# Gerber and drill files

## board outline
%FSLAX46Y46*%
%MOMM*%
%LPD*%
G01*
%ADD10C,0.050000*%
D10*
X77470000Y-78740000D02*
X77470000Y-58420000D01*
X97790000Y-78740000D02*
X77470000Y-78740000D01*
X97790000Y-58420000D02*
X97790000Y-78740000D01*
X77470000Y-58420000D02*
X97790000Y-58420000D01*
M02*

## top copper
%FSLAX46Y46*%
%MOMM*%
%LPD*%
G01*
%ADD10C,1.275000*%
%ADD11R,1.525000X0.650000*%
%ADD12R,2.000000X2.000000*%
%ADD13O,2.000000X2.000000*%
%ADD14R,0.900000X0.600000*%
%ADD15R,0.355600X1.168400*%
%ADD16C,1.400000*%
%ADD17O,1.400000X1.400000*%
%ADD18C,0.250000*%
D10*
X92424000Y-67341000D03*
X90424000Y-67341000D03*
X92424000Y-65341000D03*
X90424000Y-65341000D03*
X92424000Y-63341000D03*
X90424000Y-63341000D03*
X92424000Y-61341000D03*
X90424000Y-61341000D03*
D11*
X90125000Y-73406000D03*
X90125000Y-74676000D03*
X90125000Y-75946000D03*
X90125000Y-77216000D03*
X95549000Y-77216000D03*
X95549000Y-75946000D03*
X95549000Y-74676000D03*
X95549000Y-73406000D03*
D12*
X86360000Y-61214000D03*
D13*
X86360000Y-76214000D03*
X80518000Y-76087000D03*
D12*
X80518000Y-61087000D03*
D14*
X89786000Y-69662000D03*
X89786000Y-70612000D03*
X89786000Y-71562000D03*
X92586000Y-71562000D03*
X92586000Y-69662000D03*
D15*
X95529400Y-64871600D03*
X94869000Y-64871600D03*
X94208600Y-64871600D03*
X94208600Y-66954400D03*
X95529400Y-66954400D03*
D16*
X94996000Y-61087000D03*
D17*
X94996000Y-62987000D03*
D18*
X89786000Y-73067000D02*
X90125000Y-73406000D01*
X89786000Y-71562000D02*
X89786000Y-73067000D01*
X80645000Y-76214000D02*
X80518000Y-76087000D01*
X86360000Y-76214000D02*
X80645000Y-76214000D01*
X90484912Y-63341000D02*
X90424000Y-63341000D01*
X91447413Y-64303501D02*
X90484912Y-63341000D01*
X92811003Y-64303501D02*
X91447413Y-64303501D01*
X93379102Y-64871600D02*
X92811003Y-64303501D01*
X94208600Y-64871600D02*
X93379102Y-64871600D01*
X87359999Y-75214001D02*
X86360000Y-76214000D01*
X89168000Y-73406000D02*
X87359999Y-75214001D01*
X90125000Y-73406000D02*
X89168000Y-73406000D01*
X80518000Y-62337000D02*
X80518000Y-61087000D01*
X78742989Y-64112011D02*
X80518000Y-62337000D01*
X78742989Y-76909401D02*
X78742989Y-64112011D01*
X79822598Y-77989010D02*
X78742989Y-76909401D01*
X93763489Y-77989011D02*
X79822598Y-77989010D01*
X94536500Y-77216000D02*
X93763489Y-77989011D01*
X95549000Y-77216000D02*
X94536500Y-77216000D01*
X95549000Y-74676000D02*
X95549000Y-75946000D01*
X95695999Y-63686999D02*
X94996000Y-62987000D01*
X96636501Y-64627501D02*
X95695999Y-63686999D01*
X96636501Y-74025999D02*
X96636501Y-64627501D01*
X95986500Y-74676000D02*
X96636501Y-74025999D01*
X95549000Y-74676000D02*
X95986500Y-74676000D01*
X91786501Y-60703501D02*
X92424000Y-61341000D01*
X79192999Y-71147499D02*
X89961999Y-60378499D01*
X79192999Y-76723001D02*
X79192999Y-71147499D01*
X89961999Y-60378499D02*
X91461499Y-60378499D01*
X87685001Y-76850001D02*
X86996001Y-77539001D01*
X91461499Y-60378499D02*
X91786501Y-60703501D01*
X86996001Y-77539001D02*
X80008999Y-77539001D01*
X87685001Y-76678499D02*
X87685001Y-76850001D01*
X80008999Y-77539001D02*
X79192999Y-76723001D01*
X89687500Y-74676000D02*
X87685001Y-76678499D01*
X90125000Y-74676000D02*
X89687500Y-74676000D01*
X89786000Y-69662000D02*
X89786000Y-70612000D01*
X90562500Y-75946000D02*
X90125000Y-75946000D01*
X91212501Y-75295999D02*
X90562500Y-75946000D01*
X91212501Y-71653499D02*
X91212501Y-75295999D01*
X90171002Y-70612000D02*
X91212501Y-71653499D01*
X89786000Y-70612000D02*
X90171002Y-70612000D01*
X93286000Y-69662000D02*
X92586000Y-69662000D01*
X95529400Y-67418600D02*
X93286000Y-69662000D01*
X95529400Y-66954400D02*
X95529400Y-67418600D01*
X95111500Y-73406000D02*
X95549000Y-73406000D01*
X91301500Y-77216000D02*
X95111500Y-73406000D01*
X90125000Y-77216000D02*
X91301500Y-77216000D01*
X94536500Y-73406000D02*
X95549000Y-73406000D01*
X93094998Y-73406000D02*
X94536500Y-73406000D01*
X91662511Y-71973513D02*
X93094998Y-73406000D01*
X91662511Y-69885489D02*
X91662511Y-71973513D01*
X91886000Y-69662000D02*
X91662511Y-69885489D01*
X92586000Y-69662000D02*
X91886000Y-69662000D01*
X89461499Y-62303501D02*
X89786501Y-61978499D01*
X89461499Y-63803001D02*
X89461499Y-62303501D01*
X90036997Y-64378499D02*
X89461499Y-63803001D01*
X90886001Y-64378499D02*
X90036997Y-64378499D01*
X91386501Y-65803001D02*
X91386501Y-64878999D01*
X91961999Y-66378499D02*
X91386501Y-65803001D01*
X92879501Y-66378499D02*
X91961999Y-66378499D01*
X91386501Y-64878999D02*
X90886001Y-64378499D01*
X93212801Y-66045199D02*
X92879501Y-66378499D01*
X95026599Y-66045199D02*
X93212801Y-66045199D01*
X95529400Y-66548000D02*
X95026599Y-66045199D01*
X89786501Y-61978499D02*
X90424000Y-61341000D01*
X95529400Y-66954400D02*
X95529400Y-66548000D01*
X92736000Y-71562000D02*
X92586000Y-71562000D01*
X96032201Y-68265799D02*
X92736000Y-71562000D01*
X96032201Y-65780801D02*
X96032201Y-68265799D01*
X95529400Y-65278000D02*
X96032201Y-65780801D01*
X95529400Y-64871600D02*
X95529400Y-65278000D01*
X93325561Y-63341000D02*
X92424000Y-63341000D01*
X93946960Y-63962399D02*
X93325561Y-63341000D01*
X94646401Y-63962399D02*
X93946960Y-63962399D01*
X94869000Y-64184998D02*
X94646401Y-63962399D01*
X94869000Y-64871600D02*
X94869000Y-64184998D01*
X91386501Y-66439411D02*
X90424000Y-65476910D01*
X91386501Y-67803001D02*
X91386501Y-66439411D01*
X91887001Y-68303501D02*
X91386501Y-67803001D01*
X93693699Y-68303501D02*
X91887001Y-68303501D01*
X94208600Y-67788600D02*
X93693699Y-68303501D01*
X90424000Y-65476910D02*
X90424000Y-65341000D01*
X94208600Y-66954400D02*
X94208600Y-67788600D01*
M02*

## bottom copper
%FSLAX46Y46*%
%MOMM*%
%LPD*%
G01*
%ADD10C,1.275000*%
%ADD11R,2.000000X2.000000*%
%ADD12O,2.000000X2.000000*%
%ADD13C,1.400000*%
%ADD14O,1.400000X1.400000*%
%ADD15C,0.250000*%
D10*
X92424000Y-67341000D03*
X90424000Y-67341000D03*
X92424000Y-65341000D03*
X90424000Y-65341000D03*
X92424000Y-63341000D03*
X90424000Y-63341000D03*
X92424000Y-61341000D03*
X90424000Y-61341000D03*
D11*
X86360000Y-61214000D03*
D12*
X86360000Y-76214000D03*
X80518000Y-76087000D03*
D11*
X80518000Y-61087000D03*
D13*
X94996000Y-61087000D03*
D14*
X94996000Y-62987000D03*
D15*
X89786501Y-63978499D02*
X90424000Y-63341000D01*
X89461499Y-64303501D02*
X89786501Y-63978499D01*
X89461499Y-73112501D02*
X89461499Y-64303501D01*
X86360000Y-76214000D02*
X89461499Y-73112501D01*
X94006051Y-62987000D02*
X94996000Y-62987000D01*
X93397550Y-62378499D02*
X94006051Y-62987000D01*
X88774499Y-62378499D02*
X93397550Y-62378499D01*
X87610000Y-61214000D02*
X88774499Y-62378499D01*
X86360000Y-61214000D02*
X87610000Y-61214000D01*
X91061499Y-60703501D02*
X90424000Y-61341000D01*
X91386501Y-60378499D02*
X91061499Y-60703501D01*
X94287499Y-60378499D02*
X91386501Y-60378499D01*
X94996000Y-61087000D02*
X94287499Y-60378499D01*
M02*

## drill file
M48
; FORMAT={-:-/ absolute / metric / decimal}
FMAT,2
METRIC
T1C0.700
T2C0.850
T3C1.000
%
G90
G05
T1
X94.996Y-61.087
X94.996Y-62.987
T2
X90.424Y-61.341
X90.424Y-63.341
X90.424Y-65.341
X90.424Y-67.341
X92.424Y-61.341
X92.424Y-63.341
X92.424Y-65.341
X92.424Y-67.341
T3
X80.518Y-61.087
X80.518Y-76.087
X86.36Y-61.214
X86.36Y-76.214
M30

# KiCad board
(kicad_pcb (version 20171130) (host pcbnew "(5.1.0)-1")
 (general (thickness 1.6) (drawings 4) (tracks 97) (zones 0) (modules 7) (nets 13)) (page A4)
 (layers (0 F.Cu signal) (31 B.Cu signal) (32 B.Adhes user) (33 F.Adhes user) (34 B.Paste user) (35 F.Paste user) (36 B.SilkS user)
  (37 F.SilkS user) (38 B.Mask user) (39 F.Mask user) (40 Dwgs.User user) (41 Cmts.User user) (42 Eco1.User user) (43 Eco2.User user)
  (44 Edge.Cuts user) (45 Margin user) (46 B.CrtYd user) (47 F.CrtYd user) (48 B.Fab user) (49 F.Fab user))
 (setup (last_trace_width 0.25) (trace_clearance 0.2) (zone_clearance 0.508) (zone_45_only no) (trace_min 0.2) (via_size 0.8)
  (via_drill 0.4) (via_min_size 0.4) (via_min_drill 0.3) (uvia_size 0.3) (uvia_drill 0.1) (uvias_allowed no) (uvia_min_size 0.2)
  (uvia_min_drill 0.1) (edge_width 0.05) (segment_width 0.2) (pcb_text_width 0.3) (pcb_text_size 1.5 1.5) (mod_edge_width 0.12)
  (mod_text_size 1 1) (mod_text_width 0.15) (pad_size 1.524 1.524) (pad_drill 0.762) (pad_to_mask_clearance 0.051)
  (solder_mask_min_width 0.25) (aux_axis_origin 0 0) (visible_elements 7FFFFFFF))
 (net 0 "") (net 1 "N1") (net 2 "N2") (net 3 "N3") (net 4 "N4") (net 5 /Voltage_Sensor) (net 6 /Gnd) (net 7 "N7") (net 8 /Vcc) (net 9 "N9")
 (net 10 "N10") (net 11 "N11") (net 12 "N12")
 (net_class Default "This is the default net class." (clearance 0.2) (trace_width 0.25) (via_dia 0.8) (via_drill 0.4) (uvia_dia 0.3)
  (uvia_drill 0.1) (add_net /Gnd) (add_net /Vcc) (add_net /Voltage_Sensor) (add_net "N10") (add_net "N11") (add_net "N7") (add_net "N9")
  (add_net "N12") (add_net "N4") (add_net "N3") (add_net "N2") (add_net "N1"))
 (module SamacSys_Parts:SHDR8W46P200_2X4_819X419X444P (layer F.Cu) (at 90.424 61.341 270)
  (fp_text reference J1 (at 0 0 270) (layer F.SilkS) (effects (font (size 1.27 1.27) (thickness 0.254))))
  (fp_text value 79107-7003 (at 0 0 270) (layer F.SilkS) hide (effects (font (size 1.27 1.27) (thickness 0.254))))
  (pad 8 thru_hole circle (at 6 -2 270) (size 1.275 1.275) (drill 0.85) (layers *.Cu *.Mask) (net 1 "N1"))
  (pad 7 thru_hole circle (at 6 0 270) (size 1.275 1.275) (drill 0.85) (layers *.Cu *.Mask) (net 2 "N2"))
  (pad 6 thru_hole circle (at 4 -2 270) (size 1.275 1.275) (drill 0.85) (layers *.Cu *.Mask) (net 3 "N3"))
  (pad 5 thru_hole circle (at 4 0 270) (size 1.275 1.275) (drill 0.85) (layers *.Cu *.Mask) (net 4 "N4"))
  (pad 4 thru_hole circle (at 2 -2 270) (size 1.275 1.275) (drill 0.85) (layers *.Cu *.Mask) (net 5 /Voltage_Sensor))
  (pad 3 thru_hole circle (at 2 0 270) (size 1.275 1.275) (drill 0.85) (layers *.Cu *.Mask) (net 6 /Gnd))
  (pad 2 thru_hole circle (at 0 -2 270) (size 1.275 1.275) (drill 0.85) (layers *.Cu *.Mask) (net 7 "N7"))
  (pad 1 thru_hole circle (at 0 0 270) (size 1.275 1.275) (drill 0.85) (layers *.Cu *.Mask) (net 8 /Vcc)))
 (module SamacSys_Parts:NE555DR (layer F.Cu) (at 92.837 75.311)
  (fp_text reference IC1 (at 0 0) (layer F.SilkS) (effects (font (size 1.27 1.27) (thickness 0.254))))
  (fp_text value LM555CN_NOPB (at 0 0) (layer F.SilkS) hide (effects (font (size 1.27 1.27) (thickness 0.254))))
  (pad 1 smd rect (at -2.712 -1.905 90) (size 0.65 1.525) (layers F.Cu F.Paste) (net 6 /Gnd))
  (pad 2 smd rect (at -2.712 -0.635 90) (size 0.65 1.525) (layers F.Cu F.Paste) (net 7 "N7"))
  (pad 3 smd rect (at -2.712 0.635 90) (size 0.65 1.525) (layers F.Cu F.Paste) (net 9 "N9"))
  (pad 4 smd rect (at -2.712 1.905 90) (size 0.65 1.525) (layers F.Cu F.Paste) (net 8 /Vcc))
  (pad 5 smd rect (at 2.712 1.905 90) (size 0.65 1.525) (layers F.Cu F.Paste) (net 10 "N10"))
  (pad 6 smd rect (at 2.712 0.635 90) (size 0.65 1.525) (layers F.Cu F.Paste) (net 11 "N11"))
  (pad 7 smd rect (at 2.712 -0.635 90) (size 0.65 1.525) (layers F.Cu F.Paste) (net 11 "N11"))
  (pad 8 smd rect (at 2.712 -1.905 90) (size 0.65 1.525) (layers F.Cu F.Paste) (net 8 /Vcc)))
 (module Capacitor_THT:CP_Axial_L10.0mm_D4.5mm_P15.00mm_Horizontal (layer F.Cu) (at 86.36 61.214 270)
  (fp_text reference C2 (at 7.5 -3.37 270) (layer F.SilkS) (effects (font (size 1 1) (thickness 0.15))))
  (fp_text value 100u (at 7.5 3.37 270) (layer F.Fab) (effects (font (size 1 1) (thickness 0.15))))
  (pad 1 thru_hole rect (at 0 0 270) (size 2 2) (drill 1) (layers *.Cu *.Mask) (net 11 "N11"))
  (pad 2 thru_hole oval (at 15 0 270) (size 2 2) (drill 1) (layers *.Cu *.Mask) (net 6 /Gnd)))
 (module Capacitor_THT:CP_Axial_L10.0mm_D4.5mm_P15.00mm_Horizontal (layer F.Cu) (at 80.518 61.087 270)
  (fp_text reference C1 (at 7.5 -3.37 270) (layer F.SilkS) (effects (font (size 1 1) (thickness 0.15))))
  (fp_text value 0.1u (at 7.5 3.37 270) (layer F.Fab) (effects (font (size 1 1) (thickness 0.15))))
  (pad 2 thru_hole oval (at 15 0 270) (size 2 2) (drill 1) (layers *.Cu *.Mask) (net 6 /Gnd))
  (pad 1 thru_hole rect (at 0 0 270) (size 2 2) (drill 1) (layers *.Cu *.Mask) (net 10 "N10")))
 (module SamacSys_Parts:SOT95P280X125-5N (layer F.Cu) (at 91.186 70.612)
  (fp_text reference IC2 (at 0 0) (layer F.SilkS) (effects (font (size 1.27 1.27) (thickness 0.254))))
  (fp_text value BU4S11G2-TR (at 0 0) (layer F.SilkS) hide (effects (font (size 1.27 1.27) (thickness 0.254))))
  (pad 1 smd rect (at -1.4 -0.95 90) (size 0.6 0.9) (layers F.Cu F.Paste F.Mask) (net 9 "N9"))
  (pad 2 smd rect (at -1.4 0 90) (size 0.6 0.9) (layers F.Cu F.Paste F.Mask) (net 9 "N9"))
  (pad 3 smd rect (at -1.4 0.95 90) (size 0.6 0.9) (layers F.Cu F.Paste F.Mask) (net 6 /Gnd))
  (pad 4 smd rect (at 1.4 0.95 90) (size 0.6 0.9) (layers F.Cu F.Paste F.Mask) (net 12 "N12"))
  (pad 5 smd rect (at 1.4 -0.95 90) (size 0.6 0.9) (layers F.Cu F.Paste F.Mask) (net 8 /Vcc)))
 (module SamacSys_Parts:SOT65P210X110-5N (layer F.Cu) (at 94.869 65.913 270)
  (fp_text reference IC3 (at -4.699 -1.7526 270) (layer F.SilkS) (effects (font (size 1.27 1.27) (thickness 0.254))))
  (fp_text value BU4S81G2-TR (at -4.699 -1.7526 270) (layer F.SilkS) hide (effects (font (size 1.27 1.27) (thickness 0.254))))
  (pad 1 smd rect (at -1.0414 -0.6604) (size 0.3556 1.1684) (layers F.Cu F.Paste F.Mask) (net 12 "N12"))
  (pad 2 smd rect (at -1.0414 0) (size 0.3556 1.1684) (layers F.Cu F.Paste F.Mask) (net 5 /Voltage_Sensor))
  (pad 3 smd rect (at -1.0414 0.6604) (size 0.3556 1.1684) (layers F.Cu F.Paste F.Mask) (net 6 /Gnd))
  (pad 4 smd rect (at 1.0414 0.6604) (size 0.3556 1.1684) (layers F.Cu F.Paste F.Mask) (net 4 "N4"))
  (pad 5 smd rect (at 1.0414 -0.6604) (size 0.3556 1.1684) (layers F.Cu F.Paste F.Mask) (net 8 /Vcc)))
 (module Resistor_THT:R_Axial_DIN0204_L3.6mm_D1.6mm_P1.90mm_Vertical (layer F.Cu) (at 94.996 61.087 270)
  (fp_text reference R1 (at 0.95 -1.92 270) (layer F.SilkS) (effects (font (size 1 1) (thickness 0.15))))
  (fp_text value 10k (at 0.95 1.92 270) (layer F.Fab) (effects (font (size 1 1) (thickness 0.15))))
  (pad 1 thru_hole circle (at 0 0 270) (size 1.4 1.4) (drill 0.7) (layers *.Cu *.Mask) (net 8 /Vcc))
  (pad 2 thru_hole oval (at 1.9 0 270) (size 1.4 1.4) (drill 0.7) (layers *.Cu *.Mask) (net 11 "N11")))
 (gr_line (start 77.47 78.74) (end 77.47 58.42) (layer Edge.Cuts) (width 0.05))
 (gr_line (start 97.79 78.74) (end 77.47 78.74) (layer Edge.Cuts) (width 0.05))
 (gr_line (start 97.79 58.42) (end 97.79 78.74) (layer Edge.Cuts) (width 0.05))
 (gr_line (start 77.47 58.42) (end 97.79 58.42) (layer Edge.Cuts) (width 0.05))
 (segment (start 89.786 73.067) (end 90.125 73.406) (width 0.25) (layer F.Cu) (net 6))
 (segment (start 89.786 71.562) (end 89.786 73.067) (width 0.25) (layer F.Cu) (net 6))
 (segment (start 80.645 76.214) (end 80.518 76.087) (width 0.25) (layer F.Cu) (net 6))
 (segment (start 86.36 76.214) (end 80.645 76.214) (width 0.25) (layer F.Cu) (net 6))
 (segment (start 89.786501 63.978499) (end 90.424 63.341) (width 0.25) (layer B.Cu) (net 6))
 (segment (start 89.461499 64.303501) (end 89.786501 63.978499) (width 0.25) (layer B.Cu) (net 6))
 (segment (start 89.461499 73.112501) (end 89.461499 64.303501) (width 0.25) (layer B.Cu) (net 6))
 (segment (start 86.36 76.214) (end 89.461499 73.112501) (width 0.25) (layer B.Cu) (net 6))
 (segment (start 90.484912 63.341) (end 90.424 63.341) (width 0.25) (layer F.Cu) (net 6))
 (segment (start 91.447413 64.303501) (end 90.484912 63.341) (width 0.25) (layer F.Cu) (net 6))
 (segment (start 92.811003 64.303501) (end 91.447413 64.303501) (width 0.25) (layer F.Cu) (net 6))
 (segment (start 93.379102 64.8716) (end 92.811003 64.303501) (width 0.25) (layer F.Cu) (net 6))
 (segment (start 94.2086 64.8716) (end 93.379102 64.8716) (width 0.25) (layer F.Cu) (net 6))
 (segment (start 87.359999 75.214001) (end 86.36 76.214) (width 0.25) (layer F.Cu) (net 6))
 (segment (start 89.168 73.406) (end 87.359999 75.214001) (width 0.25) (layer F.Cu) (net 6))
 (segment (start 90.125 73.406) (end 89.168 73.406) (width 0.25) (layer F.Cu) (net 6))
 (segment (start 80.518 62.337) (end 80.518 61.087) (width 0.25) (layer F.Cu) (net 10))
 (segment (start 78.742989 64.112011) (end 80.518 62.337) (width 0.25) (layer F.Cu) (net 10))
 (segment (start 78.742989 76.909401) (end 78.742989 64.112011) (width 0.25) (layer F.Cu) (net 10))
 (segment (start 79.822598 77.98901) (end 78.742989 76.909401) (width 0.25) (layer F.Cu) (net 10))
 (segment (start 93.763489 77.989011) (end 79.822598 77.98901) (width 0.25) (layer F.Cu) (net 10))
 (segment (start 94.5365 77.216) (end 93.763489 77.989011) (width 0.25) (layer F.Cu) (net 10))
 (segment (start 95.549 77.216) (end 94.5365 77.216) (width 0.25) (layer F.Cu) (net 10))
 (segment (start 95.549 74.676) (end 95.549 75.946) (width 0.25) (layer F.Cu) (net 11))
 (segment (start 95.695999 63.686999) (end 94.996 62.987) (width 0.25) (layer F.Cu) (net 11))
 (segment (start 96.636501 64.627501) (end 95.695999 63.686999) (width 0.25) (layer F.Cu) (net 11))
 (segment (start 96.636501 74.025999) (end 96.636501 64.627501) (width 0.25) (layer F.Cu) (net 11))
 (segment (start 95.9865 74.676) (end 96.636501 74.025999) (width 0.25) (layer F.Cu) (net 11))
 (segment (start 95.549 74.676) (end 95.9865 74.676) (width 0.25) (layer F.Cu) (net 11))
 (segment (start 94.006051 62.987) (end 94.996 62.987) (width 0.25) (layer B.Cu) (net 11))
 (segment (start 93.39755 62.378499) (end 94.006051 62.987) (width 0.25) (layer B.Cu) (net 11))
 (segment (start 88.774499 62.378499) (end 93.39755 62.378499) (width 0.25) (layer B.Cu) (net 11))
 (segment (start 87.61 61.214) (end 88.774499 62.378499) (width 0.25) (layer B.Cu) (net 11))
 (segment (start 86.36 61.214) (end 87.61 61.214) (width 0.25) (layer B.Cu) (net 11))
 (segment (start 91.786501 60.703501) (end 92.424 61.341) (width 0.25) (layer F.Cu) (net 7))
 (segment (start 79.192999 71.147499) (end 89.961999 60.378499) (width 0.25) (layer F.Cu) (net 7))
 (segment (start 79.192999 76.723001) (end 79.192999 71.147499) (width 0.25) (layer F.Cu) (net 7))
 (segment (start 89.961999 60.378499) (end 91.461499 60.378499) (width 0.25) (layer F.Cu) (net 7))
 (segment (start 87.685001 76.850001) (end 86.996001 77.539001) (width 0.25) (layer F.Cu) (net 7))
 (segment (start 91.461499 60.378499) (end 91.786501 60.703501) (width 0.25) (layer F.Cu) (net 7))
 (segment (start 86.996001 77.539001) (end 80.008999 77.539001) (width 0.25) (layer F.Cu) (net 7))
 (segment (start 87.685001 76.678499) (end 87.685001 76.850001) (width 0.25) (layer F.Cu) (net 7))
 (segment (start 80.008999 77.539001) (end 79.192999 76.723001) (width 0.25) (layer F.Cu) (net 7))
 (segment (start 89.6875 74.676) (end 87.685001 76.678499) (width 0.25) (layer F.Cu) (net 7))
 (segment (start 90.125 74.676) (end 89.6875 74.676) (width 0.25) (layer F.Cu) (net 7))
 (segment (start 89.786 69.662) (end 89.786 70.612) (width 0.25) (layer F.Cu) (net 9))
 (segment (start 90.5625 75.946) (end 90.125 75.946) (width 0.25) (layer F.Cu) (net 9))
 (segment (start 91.212501 75.295999) (end 90.5625 75.946) (width 0.25) (layer F.Cu) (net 9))
 (segment (start 91.212501 71.653499) (end 91.212501 75.295999) (width 0.25) (layer F.Cu) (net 9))
 (segment (start 90.171002 70.612) (end 91.212501 71.653499) (width 0.25) (layer F.Cu) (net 9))
 (segment (start 89.786 70.612) (end 90.171002 70.612) (width 0.25) (layer F.Cu) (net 9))
 (segment (start 93.286 69.662) (end 92.586 69.662) (width 0.25) (layer F.Cu) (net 8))
 (segment (start 95.5294 67.4186) (end 93.286 69.662) (width 0.25) (layer F.Cu) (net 8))
 (segment (start 95.5294 66.9544) (end 95.5294 67.4186) (width 0.25) (layer F.Cu) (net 8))
 (segment (start 95.1115 73.406) (end 95.549 73.406) (width 0.25) (layer F.Cu) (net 8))
 (segment (start 91.3015 77.216) (end 95.1115 73.406) (width 0.25) (layer F.Cu) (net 8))
 (segment (start 90.125 77.216) (end 91.3015 77.216) (width 0.25) (layer F.Cu) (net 8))
 (segment (start 94.5365 73.406) (end 95.549 73.406) (width 0.25) (layer F.Cu) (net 8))
 (segment (start 93.094998 73.406) (end 94.5365 73.406) (width 0.25) (layer F.Cu) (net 8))
 (segment (start 91.662511 71.973513) (end 93.094998 73.406) (width 0.25) (layer F.Cu) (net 8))
 (segment (start 91.662511 69.885489) (end 91.662511 71.973513) (width 0.25) (layer F.Cu) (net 8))
 (segment (start 91.886 69.662) (end 91.662511 69.885489) (width 0.25) (layer F.Cu) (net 8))
 (segment (start 92.586 69.662) (end 91.886 69.662) (width 0.25) (layer F.Cu) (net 8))
 (segment (start 91.061499 60.703501) (end 90.424 61.341) (width 0.25) (layer B.Cu) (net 8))
 (segment (start 91.386501 60.378499) (end 91.061499 60.703501) (width 0.25) (layer B.Cu) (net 8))
 (segment (start 94.287499 60.378499) (end 91.386501 60.378499) (width 0.25) (layer B.Cu) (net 8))
 (segment (start 94.996 61.087) (end 94.287499 60.378499) (width 0.25) (layer B.Cu) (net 8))
 (segment (start 89.461499 62.303501) (end 89.786501 61.978499) (width 0.25) (layer F.Cu) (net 8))
 (segment (start 89.461499 63.803001) (end 89.461499 62.303501) (width 0.25) (layer F.Cu) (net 8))
 (segment (start 90.036997 64.378499) (end 89.461499 63.803001) (width 0.25) (layer F.Cu) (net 8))
 (segment (start 90.886001 64.378499) (end 90.036997 64.378499) (width 0.25) (layer F.Cu) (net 8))
 (segment (start 91.386501 65.803001) (end 91.386501 64.878999) (width 0.25) (layer F.Cu) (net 8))
 (segment (start 91.961999 66.378499) (end 91.386501 65.803001) (width 0.25) (layer F.Cu) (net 8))
 (segment (start 92.879501 66.378499) (end 91.961999 66.378499) (width 0.25) (layer F.Cu) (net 8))
 (segment (start 91.386501 64.878999) (end 90.886001 64.378499) (width 0.25) (layer F.Cu) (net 8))
 (segment (start 93.212801 66.045199) (end 92.879501 66.378499) (width 0.25) (layer F.Cu) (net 8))
 (segment (start 95.026599 66.045199) (end 93.212801 66.045199) (width 0.25) (layer F.Cu) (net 8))
 (segment (start 95.5294 66.548) (end 95.026599 66.045199) (width 0.25) (layer F.Cu) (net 8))
 (segment (start 89.786501 61.978499) (end 90.424 61.341) (width 0.25) (layer F.Cu) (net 8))
 (segment (start 95.5294 66.9544) (end 95.5294 66.548) (width 0.25) (layer F.Cu) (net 8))
 (segment (start 92.736 71.562) (end 92.586 71.562) (width 0.25) (layer F.Cu) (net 12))
 (segment (start 96.032201 68.265799) (end 92.736 71.562) (width 0.25) (layer F.Cu) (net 12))
 (segment (start 96.032201 65.780801) (end 96.032201 68.265799) (width 0.25) (layer F.Cu) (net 12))
 (segment (start 95.5294 65.278) (end 96.032201 65.780801) (width 0.25) (layer F.Cu) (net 12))
 (segment (start 95.5294 64.8716) (end 95.5294 65.278) (width 0.25) (layer F.Cu) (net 12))
 (segment (start 93.325561 63.341) (end 92.424 63.341) (width 0.25) (layer F.Cu) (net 5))
 (segment (start 93.94696 63.962399) (end 93.325561 63.341) (width 0.25) (layer F.Cu) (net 5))
 (segment (start 94.646401 63.962399) (end 93.94696 63.962399) (width 0.25) (layer F.Cu) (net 5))
 (segment (start 94.869 64.184998) (end 94.646401 63.962399) (width 0.25) (layer F.Cu) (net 5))
 (segment (start 94.869 64.8716) (end 94.869 64.184998) (width 0.25) (layer F.Cu) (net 5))
 (segment (start 91.386501 66.439411) (end 90.424 65.47691) (width 0.25) (layer F.Cu) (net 4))
 (segment (start 91.386501 67.803001) (end 91.386501 66.439411) (width 0.25) (layer F.Cu) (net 4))
 (segment (start 91.887001 68.303501) (end 91.386501 67.803001) (width 0.25) (layer F.Cu) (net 4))
 (segment (start 93.693699 68.303501) (end 91.887001 68.303501) (width 0.25) (layer F.Cu) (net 4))
 (segment (start 94.2086 67.7886) (end 93.693699 68.303501) (width 0.25) (layer F.Cu) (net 4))
 (segment (start 90.424 65.47691) (end 90.424 65.341) (width 0.25) (layer F.Cu) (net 4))
 (segment (start 94.2086 66.9544) (end 94.2086 67.7886) (width 0.25) (layer F.Cu) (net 4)))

